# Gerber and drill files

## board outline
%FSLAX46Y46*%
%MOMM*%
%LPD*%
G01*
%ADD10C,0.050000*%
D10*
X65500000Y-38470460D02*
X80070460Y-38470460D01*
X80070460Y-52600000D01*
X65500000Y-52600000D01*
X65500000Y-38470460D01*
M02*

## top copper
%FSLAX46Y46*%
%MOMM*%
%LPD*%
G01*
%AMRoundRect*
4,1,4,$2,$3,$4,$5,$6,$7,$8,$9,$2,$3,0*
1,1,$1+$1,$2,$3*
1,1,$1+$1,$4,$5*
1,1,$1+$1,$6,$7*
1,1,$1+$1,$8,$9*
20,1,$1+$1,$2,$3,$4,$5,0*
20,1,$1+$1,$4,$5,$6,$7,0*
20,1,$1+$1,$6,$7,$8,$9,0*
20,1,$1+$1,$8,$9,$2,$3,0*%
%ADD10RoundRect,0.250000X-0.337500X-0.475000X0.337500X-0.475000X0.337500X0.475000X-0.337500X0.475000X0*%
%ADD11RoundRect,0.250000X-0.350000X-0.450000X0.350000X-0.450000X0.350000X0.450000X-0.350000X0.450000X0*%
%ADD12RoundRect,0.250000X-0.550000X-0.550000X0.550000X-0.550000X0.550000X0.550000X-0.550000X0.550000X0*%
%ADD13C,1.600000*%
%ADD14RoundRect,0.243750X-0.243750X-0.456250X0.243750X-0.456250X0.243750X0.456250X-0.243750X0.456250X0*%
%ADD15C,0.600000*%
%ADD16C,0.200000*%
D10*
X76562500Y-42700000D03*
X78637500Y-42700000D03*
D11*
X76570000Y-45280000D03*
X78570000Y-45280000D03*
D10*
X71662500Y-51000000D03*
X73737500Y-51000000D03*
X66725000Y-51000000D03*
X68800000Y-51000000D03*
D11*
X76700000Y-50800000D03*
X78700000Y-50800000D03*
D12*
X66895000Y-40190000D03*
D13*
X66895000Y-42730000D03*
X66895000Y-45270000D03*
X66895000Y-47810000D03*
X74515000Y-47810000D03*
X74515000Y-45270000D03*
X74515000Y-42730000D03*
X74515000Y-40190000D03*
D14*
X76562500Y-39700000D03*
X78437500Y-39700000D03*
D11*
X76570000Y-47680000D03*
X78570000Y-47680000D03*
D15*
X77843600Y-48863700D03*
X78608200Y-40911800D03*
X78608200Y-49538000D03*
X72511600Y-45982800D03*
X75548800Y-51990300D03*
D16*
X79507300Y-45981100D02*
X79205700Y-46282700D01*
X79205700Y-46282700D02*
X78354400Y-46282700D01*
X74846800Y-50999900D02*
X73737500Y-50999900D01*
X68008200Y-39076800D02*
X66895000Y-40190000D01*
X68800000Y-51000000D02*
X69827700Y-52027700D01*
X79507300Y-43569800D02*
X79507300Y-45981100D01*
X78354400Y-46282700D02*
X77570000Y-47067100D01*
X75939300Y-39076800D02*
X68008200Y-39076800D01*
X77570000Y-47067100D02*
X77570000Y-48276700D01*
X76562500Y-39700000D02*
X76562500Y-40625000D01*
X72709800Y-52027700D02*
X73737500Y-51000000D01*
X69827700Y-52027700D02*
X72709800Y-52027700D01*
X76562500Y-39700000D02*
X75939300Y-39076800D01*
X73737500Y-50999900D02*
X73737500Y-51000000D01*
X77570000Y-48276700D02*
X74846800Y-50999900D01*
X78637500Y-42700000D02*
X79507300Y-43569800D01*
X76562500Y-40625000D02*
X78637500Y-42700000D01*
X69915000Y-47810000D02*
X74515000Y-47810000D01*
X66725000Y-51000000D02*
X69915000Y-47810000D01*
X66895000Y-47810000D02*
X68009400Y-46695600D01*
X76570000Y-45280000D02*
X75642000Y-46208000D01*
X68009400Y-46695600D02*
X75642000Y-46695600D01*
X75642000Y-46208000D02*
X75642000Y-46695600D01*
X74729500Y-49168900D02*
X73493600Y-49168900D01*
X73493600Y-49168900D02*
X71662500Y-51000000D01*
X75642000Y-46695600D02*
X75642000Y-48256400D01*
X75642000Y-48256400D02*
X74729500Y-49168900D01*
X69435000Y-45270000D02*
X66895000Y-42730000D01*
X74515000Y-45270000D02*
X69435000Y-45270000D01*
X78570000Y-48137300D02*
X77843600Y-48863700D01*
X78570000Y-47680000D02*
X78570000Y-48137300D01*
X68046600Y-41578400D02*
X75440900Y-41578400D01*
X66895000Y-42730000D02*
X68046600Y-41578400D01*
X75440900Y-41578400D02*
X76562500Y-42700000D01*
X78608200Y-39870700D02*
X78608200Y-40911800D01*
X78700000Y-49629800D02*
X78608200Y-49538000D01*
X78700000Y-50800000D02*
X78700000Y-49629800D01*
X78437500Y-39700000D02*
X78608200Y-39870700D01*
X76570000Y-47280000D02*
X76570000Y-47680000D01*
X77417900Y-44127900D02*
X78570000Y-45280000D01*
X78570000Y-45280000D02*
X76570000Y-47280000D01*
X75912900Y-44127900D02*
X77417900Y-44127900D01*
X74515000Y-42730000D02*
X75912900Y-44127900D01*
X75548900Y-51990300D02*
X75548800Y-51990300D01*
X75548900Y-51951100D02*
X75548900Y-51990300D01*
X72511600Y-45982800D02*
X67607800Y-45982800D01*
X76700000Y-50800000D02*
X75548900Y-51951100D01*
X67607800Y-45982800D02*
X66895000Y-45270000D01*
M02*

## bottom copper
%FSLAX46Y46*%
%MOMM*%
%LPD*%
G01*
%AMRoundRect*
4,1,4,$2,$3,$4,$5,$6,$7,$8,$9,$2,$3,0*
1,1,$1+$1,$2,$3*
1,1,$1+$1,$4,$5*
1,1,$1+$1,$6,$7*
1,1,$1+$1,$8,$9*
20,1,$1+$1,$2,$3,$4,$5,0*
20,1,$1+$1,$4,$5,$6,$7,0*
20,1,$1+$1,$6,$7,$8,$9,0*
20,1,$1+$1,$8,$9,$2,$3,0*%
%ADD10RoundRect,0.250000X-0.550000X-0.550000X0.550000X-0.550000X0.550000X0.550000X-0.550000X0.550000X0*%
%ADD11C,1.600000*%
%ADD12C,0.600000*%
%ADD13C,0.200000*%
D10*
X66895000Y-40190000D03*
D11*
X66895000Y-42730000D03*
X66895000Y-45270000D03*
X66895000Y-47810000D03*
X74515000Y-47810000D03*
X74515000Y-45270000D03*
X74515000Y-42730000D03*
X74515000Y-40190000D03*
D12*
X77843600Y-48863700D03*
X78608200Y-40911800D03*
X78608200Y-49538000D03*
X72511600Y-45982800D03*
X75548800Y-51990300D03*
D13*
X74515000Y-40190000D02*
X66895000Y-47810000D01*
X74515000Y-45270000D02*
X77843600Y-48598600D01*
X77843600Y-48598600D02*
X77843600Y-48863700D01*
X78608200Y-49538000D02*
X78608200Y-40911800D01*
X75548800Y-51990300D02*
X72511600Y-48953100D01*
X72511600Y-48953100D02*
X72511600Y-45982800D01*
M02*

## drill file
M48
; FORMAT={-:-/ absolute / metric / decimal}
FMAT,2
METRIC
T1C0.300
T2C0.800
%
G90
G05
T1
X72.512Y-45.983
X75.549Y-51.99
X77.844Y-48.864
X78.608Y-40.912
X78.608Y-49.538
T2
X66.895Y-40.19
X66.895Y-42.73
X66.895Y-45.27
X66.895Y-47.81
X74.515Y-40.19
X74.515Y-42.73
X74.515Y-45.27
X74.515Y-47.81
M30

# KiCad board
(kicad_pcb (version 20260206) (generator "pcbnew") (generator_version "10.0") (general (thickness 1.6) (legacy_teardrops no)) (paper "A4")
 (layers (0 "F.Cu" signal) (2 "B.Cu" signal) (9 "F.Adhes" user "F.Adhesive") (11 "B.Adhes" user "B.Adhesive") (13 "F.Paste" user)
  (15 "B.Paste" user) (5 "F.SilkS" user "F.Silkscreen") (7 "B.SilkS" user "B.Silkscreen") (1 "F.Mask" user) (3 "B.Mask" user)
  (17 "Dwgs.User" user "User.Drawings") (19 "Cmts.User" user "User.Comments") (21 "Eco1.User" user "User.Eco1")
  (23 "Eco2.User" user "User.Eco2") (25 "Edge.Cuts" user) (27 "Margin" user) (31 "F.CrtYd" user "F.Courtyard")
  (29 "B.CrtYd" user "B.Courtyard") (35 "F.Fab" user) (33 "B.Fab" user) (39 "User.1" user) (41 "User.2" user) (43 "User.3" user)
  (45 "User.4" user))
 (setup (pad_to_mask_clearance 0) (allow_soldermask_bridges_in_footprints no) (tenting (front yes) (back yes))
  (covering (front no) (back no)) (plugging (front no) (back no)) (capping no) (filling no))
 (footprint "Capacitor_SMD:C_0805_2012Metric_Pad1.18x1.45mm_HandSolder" (layer "F.Cu") (at 77.6 42.7)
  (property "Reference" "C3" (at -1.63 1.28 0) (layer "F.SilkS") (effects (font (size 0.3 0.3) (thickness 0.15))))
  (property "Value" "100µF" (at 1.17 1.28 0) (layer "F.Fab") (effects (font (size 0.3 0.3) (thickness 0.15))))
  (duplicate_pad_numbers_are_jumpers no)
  (pad "1" smd roundrect (at -1.0375 0) (size 1.175 1.45) (layers "F.Cu" "F.Mask" "F.Paste") (roundrect_rratio 0.212766) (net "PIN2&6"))
  (pad "2" smd roundrect (at 1.0375 0) (size 1.175 1.45) (layers "F.Cu" "F.Mask" "F.Paste") (roundrect_rratio 0.212766) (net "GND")))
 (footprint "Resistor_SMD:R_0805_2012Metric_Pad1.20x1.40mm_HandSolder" (layer "F.Cu") (at 77.57 45.28)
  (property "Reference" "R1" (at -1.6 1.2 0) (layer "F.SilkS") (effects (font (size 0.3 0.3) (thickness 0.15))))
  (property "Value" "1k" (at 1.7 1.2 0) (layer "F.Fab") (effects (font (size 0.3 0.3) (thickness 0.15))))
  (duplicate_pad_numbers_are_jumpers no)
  (pad "1" smd roundrect (at -1 0) (size 1.2 1.4) (layers "F.Cu" "F.Mask" "F.Paste") (roundrect_rratio 0.208333) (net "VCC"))
  (pad "2" smd roundrect (at 1 0) (size 1.2 1.4) (layers "F.Cu" "F.Mask" "F.Paste") (roundrect_rratio 0.208333) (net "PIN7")))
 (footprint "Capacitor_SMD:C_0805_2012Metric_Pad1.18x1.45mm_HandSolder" (layer "F.Cu") (at 72.7 51)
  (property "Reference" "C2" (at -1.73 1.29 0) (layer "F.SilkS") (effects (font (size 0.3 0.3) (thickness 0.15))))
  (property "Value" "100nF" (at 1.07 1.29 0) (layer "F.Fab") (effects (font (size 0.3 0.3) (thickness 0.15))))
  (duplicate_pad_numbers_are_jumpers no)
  (pad "1" smd roundrect (at -1.0375 0) (size 1.175 1.45) (layers "F.Cu" "F.Mask" "F.Paste") (roundrect_rratio 0.212766) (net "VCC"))
  (pad "2" smd roundrect (at 1.0375 0) (size 1.175 1.45) (layers "F.Cu" "F.Mask" "F.Paste") (roundrect_rratio 0.212766) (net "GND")))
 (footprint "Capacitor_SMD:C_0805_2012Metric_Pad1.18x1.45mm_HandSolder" (layer "F.Cu") (at 67.7625 51)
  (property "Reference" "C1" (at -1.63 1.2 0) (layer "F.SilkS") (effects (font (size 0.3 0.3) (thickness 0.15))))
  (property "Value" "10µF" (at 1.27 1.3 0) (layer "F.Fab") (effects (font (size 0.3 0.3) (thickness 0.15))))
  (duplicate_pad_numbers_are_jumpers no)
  (pad "1" smd roundrect (at -1.0375 0) (size 1.175 1.45) (layers "F.Cu" "F.Mask" "F.Paste") (roundrect_rratio 0.212766) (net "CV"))
  (pad "2" smd roundrect (at 1.0375 0) (size 1.175 1.45) (layers "F.Cu" "F.Mask" "F.Paste") (roundrect_rratio 0.212766) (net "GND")))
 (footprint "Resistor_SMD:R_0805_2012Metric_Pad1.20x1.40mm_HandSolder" (layer "F.Cu") (at 77.7 50.8)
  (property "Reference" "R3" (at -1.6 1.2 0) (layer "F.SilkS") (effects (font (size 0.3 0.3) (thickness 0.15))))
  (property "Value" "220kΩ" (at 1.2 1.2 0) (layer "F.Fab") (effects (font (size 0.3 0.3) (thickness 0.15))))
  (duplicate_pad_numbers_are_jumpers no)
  (pad "1" smd roundrect (at -1 0) (size 1.2 1.4) (layers "F.Cu" "F.Mask" "F.Paste") (roundrect_rratio 0.208333) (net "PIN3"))
  (pad "2" smd roundrect (at 1 0) (size 1.2 1.4) (layers "F.Cu" "F.Mask" "F.Paste") (roundrect_rratio 0.208333) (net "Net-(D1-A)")))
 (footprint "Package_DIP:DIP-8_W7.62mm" (layer "F.Cu") (at 66.895 40.19)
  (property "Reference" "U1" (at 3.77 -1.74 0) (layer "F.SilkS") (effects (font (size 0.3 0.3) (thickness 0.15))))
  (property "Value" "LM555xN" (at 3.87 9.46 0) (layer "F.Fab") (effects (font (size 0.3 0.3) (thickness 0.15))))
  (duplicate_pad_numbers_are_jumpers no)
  (pad "1" thru_hole roundrect (at 0 0) (size 1.6 1.6) (drill 0.8) (layers "*.Cu" "*.Mask") (remove_unused_layers no)
   (roundrect_rratio 0.15625) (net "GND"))
  (pad "2" thru_hole circle (at 0 2.54) (size 1.6 1.6) (drill 0.8) (layers "*.Cu" "*.Mask") (remove_unused_layers no) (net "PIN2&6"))
  (pad "3" thru_hole circle (at 0 5.08) (size 1.6 1.6) (drill 0.8) (layers "*.Cu" "*.Mask") (remove_unused_layers no) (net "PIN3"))
  (pad "4" thru_hole circle (at 0 7.62) (size 1.6 1.6) (drill 0.8) (layers "*.Cu" "*.Mask") (remove_unused_layers no) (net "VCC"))
  (pad "5" thru_hole circle (at 7.62 7.62) (size 1.6 1.6) (drill 0.8) (layers "*.Cu" "*.Mask") (remove_unused_layers no) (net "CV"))
  (pad "6" thru_hole circle (at 7.62 5.08) (size 1.6 1.6) (drill 0.8) (layers "*.Cu" "*.Mask") (remove_unused_layers no) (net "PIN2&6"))
  (pad "7" thru_hole circle (at 7.62 2.54) (size 1.6 1.6) (drill 0.8) (layers "*.Cu" "*.Mask") (remove_unused_layers no) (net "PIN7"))
  (pad "8" thru_hole circle (at 7.62 0) (size 1.6 1.6) (drill 0.8) (layers "*.Cu" "*.Mask") (remove_unused_layers no) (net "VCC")))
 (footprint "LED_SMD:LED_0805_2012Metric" (layer "F.Cu") (at 77.5 39.7)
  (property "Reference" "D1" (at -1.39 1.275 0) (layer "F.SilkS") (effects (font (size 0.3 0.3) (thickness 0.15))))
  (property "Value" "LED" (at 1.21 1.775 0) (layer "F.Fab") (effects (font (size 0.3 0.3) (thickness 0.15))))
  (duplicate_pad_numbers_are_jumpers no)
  (pad "1" smd roundrect (at -0.9375 0) (size 0.975 1.4) (layers "F.Cu" "F.Mask" "F.Paste") (roundrect_rratio 0.25) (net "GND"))
  (pad "2" smd roundrect (at 0.9375 0) (size 0.975 1.4) (layers "F.Cu" "F.Mask" "F.Paste") (roundrect_rratio 0.25) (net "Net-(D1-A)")))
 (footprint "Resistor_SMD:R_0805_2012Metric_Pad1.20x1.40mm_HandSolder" (layer "F.Cu") (at 77.57 47.68)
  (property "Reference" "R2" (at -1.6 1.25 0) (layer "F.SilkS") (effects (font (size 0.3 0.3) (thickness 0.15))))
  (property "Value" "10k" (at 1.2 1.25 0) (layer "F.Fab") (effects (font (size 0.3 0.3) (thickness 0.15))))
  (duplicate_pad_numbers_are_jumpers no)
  (pad "1" smd roundrect (at -1 0) (size 1.2 1.4) (layers "F.Cu" "F.Mask" "F.Paste") (roundrect_rratio 0.208333) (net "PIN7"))
  (pad "2" smd roundrect (at 1 0) (size 1.2 1.4) (layers "F.Cu" "F.Mask" "F.Paste") (roundrect_rratio 0.208333) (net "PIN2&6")))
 (gr_rect (start 65.5 38.47046) (end 80.07046 52.6) (stroke (width 0.05) (type default)) (fill no) (layer "Edge.Cuts"))
 (segment (start 79.5073 45.9811) (end 79.2057 46.2827) (width 0.2) (layer "F.Cu") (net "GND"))
 (segment (start 79.2057 46.2827) (end 78.3544 46.2827) (width 0.2) (layer "F.Cu") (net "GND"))
 (segment (start 74.8468 50.9999) (end 73.7375 50.9999) (width 0.2) (layer "F.Cu") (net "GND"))
 (segment (start 68.0082 39.0768) (end 66.895 40.19) (width 0.2) (layer "F.Cu") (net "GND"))
 (segment (start 68.8 51) (end 69.8277 52.0277) (width 0.2) (layer "F.Cu") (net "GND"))
 (segment (start 79.5073 43.5698) (end 79.5073 45.9811) (width 0.2) (layer "F.Cu") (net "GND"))
 (segment (start 78.3544 46.2827) (end 77.57 47.0671) (width 0.2) (layer "F.Cu") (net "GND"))
 (segment (start 75.9393 39.0768) (end 68.0082 39.0768) (width 0.2) (layer "F.Cu") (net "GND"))
 (segment (start 77.57 47.0671) (end 77.57 48.2767) (width 0.2) (layer "F.Cu") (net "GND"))
 (segment (start 76.5625 39.7) (end 76.5625 40.625) (width 0.2) (layer "F.Cu") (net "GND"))
 (segment (start 72.7098 52.0277) (end 73.7375 51) (width 0.2) (layer "F.Cu") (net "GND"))
 (segment (start 69.8277 52.0277) (end 72.7098 52.0277) (width 0.2) (layer "F.Cu") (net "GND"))
 (segment (start 76.5625 39.7) (end 75.9393 39.0768) (width 0.2) (layer "F.Cu") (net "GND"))
 (segment (start 73.7375 50.9999) (end 73.7375 51) (width 0.2) (layer "F.Cu") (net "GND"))
 (segment (start 77.57 48.2767) (end 74.8468 50.9999) (width 0.2) (layer "F.Cu") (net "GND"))
 (segment (start 78.6375 42.7) (end 79.5073 43.5698) (width 0.2) (layer "F.Cu") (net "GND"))
 (segment (start 76.5625 40.625) (end 78.6375 42.7) (width 0.2) (layer "F.Cu") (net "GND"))
 (segment (start 69.915 47.81) (end 74.515 47.81) (width 0.2) (layer "F.Cu") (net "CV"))
 (segment (start 66.725 51) (end 69.915 47.81) (width 0.2) (layer "F.Cu") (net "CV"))
 (segment (start 66.895 47.81) (end 68.0094 46.6956) (width 0.2) (layer "F.Cu") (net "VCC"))
 (segment (start 76.57 45.28) (end 75.642 46.208) (width 0.2) (layer "F.Cu") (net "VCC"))
 (segment (start 68.0094 46.6956) (end 75.642 46.6956) (width 0.2) (layer "F.Cu") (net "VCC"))
 (segment (start 75.642 46.208) (end 75.642 46.6956) (width 0.2) (layer "F.Cu") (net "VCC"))
 (segment (start 74.7295 49.1689) (end 73.4936 49.1689) (width 0.2) (layer "F.Cu") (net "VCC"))
 (segment (start 73.4936 49.1689) (end 71.6625 51) (width 0.2) (layer "F.Cu") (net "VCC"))
 (segment (start 75.642 46.6956) (end 75.642 48.2564) (width 0.2) (layer "F.Cu") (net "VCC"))
 (segment (start 75.642 48.2564) (end 74.7295 49.1689) (width 0.2) (layer "F.Cu") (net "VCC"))
 (segment (start 74.515 40.19) (end 66.895 47.81) (width 0.2) (layer "B.Cu") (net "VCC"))
 (segment (start 69.435 45.27) (end 66.895 42.73) (width 0.2) (layer "F.Cu") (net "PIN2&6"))
 (segment (start 74.515 45.27) (end 69.435 45.27) (width 0.2) (layer "F.Cu") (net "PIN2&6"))
 (segment (start 78.57 48.1373) (end 77.8436 48.8637) (width 0.2) (layer "F.Cu") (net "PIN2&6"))
 (segment (start 78.57 47.68) (end 78.57 48.1373) (width 0.2) (layer "F.Cu") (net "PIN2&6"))
 (segment (start 68.0466 41.5784) (end 75.4409 41.5784) (width 0.2) (layer "F.Cu") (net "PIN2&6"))
 (segment (start 66.895 42.73) (end 68.0466 41.5784) (width 0.2) (layer "F.Cu") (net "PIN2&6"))
 (segment (start 75.4409 41.5784) (end 76.5625 42.7) (width 0.2) (layer "F.Cu") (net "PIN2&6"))
 (via (at 77.8436 48.8637) (size 0.6) (drill 0.3) (layers "F.Cu" "B.Cu") (capping no) (covering (front no) (back no))
  (plugging (front no) (back no)) (filling no) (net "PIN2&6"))
 (segment (start 74.515 45.27) (end 77.8436 48.5986) (width 0.2) (layer "B.Cu") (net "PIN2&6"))
 (segment (start 77.8436 48.5986) (end 77.8436 48.8637) (width 0.2) (layer "B.Cu") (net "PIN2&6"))
 (segment (start 78.6082 39.8707) (end 78.6082 40.9118) (width 0.2) (layer "F.Cu") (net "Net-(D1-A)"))
 (segment (start 78.7 49.6298) (end 78.6082 49.538) (width 0.2) (layer "F.Cu") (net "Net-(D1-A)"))
 (segment (start 78.7 50.8) (end 78.7 49.6298) (width 0.2) (layer "F.Cu") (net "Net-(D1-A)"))
 (segment (start 78.4375 39.7) (end 78.6082 39.8707) (width 0.2) (layer "F.Cu") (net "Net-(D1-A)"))
 (via (at 78.6082 40.9118) (size 0.6) (drill 0.3) (layers "F.Cu" "B.Cu") (capping no) (covering (front no) (back no))
  (plugging (front no) (back no)) (filling no) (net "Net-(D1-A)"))
 (via (at 78.6082 49.538) (size 0.6) (drill 0.3) (layers "F.Cu" "B.Cu") (capping no) (covering (front no) (back no))
  (plugging (front no) (back no)) (filling no) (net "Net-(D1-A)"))
 (segment (start 78.6082 49.538) (end 78.6082 40.9118) (width 0.2) (layer "B.Cu") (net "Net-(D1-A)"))
 (segment (start 76.57 47.28) (end 76.57 47.68) (width 0.2) (layer "F.Cu") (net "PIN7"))
 (segment (start 77.4179 44.1279) (end 78.57 45.28) (width 0.2) (layer "F.Cu") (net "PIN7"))
 (segment (start 78.57 45.28) (end 76.57 47.28) (width 0.2) (layer "F.Cu") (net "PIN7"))
 (segment (start 75.9129 44.1279) (end 77.4179 44.1279) (width 0.2) (layer "F.Cu") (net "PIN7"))
 (segment (start 74.515 42.73) (end 75.9129 44.1279) (width 0.2) (layer "F.Cu") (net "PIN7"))
 (segment (start 75.5489 51.9903) (end 75.5488 51.9903) (width 0.2) (layer "F.Cu") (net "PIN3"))
 (segment (start 75.5489 51.9511) (end 75.5489 51.9903) (width 0.2) (layer "F.Cu") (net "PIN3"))
 (segment (start 72.5116 45.9828) (end 67.6078 45.9828) (width 0.2) (layer "F.Cu") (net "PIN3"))
 (segment (start 76.7 50.8) (end 75.5489 51.9511) (width 0.2) (layer "F.Cu") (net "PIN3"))
 (segment (start 67.6078 45.9828) (end 66.895 45.27) (width 0.2) (layer "F.Cu") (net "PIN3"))
 (via (at 72.5116 45.9828) (size 0.6) (drill 0.3) (layers "F.Cu" "B.Cu") (capping no) (covering (front no) (back no))
  (plugging (front no) (back no)) (filling no) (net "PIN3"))
 (via (at 75.5488 51.9903) (size 0.6) (drill 0.3) (layers "F.Cu" "B.Cu") (capping no) (covering (front no) (back no))
  (plugging (front no) (back no)) (filling no) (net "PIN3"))
 (segment (start 75.5488 51.9903) (end 72.5116 48.9531) (width 0.2) (layer "B.Cu") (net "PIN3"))
 (segment (start 72.5116 48.9531) (end 72.5116 45.9828) (width 0.2) (layer "B.Cu") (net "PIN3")))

